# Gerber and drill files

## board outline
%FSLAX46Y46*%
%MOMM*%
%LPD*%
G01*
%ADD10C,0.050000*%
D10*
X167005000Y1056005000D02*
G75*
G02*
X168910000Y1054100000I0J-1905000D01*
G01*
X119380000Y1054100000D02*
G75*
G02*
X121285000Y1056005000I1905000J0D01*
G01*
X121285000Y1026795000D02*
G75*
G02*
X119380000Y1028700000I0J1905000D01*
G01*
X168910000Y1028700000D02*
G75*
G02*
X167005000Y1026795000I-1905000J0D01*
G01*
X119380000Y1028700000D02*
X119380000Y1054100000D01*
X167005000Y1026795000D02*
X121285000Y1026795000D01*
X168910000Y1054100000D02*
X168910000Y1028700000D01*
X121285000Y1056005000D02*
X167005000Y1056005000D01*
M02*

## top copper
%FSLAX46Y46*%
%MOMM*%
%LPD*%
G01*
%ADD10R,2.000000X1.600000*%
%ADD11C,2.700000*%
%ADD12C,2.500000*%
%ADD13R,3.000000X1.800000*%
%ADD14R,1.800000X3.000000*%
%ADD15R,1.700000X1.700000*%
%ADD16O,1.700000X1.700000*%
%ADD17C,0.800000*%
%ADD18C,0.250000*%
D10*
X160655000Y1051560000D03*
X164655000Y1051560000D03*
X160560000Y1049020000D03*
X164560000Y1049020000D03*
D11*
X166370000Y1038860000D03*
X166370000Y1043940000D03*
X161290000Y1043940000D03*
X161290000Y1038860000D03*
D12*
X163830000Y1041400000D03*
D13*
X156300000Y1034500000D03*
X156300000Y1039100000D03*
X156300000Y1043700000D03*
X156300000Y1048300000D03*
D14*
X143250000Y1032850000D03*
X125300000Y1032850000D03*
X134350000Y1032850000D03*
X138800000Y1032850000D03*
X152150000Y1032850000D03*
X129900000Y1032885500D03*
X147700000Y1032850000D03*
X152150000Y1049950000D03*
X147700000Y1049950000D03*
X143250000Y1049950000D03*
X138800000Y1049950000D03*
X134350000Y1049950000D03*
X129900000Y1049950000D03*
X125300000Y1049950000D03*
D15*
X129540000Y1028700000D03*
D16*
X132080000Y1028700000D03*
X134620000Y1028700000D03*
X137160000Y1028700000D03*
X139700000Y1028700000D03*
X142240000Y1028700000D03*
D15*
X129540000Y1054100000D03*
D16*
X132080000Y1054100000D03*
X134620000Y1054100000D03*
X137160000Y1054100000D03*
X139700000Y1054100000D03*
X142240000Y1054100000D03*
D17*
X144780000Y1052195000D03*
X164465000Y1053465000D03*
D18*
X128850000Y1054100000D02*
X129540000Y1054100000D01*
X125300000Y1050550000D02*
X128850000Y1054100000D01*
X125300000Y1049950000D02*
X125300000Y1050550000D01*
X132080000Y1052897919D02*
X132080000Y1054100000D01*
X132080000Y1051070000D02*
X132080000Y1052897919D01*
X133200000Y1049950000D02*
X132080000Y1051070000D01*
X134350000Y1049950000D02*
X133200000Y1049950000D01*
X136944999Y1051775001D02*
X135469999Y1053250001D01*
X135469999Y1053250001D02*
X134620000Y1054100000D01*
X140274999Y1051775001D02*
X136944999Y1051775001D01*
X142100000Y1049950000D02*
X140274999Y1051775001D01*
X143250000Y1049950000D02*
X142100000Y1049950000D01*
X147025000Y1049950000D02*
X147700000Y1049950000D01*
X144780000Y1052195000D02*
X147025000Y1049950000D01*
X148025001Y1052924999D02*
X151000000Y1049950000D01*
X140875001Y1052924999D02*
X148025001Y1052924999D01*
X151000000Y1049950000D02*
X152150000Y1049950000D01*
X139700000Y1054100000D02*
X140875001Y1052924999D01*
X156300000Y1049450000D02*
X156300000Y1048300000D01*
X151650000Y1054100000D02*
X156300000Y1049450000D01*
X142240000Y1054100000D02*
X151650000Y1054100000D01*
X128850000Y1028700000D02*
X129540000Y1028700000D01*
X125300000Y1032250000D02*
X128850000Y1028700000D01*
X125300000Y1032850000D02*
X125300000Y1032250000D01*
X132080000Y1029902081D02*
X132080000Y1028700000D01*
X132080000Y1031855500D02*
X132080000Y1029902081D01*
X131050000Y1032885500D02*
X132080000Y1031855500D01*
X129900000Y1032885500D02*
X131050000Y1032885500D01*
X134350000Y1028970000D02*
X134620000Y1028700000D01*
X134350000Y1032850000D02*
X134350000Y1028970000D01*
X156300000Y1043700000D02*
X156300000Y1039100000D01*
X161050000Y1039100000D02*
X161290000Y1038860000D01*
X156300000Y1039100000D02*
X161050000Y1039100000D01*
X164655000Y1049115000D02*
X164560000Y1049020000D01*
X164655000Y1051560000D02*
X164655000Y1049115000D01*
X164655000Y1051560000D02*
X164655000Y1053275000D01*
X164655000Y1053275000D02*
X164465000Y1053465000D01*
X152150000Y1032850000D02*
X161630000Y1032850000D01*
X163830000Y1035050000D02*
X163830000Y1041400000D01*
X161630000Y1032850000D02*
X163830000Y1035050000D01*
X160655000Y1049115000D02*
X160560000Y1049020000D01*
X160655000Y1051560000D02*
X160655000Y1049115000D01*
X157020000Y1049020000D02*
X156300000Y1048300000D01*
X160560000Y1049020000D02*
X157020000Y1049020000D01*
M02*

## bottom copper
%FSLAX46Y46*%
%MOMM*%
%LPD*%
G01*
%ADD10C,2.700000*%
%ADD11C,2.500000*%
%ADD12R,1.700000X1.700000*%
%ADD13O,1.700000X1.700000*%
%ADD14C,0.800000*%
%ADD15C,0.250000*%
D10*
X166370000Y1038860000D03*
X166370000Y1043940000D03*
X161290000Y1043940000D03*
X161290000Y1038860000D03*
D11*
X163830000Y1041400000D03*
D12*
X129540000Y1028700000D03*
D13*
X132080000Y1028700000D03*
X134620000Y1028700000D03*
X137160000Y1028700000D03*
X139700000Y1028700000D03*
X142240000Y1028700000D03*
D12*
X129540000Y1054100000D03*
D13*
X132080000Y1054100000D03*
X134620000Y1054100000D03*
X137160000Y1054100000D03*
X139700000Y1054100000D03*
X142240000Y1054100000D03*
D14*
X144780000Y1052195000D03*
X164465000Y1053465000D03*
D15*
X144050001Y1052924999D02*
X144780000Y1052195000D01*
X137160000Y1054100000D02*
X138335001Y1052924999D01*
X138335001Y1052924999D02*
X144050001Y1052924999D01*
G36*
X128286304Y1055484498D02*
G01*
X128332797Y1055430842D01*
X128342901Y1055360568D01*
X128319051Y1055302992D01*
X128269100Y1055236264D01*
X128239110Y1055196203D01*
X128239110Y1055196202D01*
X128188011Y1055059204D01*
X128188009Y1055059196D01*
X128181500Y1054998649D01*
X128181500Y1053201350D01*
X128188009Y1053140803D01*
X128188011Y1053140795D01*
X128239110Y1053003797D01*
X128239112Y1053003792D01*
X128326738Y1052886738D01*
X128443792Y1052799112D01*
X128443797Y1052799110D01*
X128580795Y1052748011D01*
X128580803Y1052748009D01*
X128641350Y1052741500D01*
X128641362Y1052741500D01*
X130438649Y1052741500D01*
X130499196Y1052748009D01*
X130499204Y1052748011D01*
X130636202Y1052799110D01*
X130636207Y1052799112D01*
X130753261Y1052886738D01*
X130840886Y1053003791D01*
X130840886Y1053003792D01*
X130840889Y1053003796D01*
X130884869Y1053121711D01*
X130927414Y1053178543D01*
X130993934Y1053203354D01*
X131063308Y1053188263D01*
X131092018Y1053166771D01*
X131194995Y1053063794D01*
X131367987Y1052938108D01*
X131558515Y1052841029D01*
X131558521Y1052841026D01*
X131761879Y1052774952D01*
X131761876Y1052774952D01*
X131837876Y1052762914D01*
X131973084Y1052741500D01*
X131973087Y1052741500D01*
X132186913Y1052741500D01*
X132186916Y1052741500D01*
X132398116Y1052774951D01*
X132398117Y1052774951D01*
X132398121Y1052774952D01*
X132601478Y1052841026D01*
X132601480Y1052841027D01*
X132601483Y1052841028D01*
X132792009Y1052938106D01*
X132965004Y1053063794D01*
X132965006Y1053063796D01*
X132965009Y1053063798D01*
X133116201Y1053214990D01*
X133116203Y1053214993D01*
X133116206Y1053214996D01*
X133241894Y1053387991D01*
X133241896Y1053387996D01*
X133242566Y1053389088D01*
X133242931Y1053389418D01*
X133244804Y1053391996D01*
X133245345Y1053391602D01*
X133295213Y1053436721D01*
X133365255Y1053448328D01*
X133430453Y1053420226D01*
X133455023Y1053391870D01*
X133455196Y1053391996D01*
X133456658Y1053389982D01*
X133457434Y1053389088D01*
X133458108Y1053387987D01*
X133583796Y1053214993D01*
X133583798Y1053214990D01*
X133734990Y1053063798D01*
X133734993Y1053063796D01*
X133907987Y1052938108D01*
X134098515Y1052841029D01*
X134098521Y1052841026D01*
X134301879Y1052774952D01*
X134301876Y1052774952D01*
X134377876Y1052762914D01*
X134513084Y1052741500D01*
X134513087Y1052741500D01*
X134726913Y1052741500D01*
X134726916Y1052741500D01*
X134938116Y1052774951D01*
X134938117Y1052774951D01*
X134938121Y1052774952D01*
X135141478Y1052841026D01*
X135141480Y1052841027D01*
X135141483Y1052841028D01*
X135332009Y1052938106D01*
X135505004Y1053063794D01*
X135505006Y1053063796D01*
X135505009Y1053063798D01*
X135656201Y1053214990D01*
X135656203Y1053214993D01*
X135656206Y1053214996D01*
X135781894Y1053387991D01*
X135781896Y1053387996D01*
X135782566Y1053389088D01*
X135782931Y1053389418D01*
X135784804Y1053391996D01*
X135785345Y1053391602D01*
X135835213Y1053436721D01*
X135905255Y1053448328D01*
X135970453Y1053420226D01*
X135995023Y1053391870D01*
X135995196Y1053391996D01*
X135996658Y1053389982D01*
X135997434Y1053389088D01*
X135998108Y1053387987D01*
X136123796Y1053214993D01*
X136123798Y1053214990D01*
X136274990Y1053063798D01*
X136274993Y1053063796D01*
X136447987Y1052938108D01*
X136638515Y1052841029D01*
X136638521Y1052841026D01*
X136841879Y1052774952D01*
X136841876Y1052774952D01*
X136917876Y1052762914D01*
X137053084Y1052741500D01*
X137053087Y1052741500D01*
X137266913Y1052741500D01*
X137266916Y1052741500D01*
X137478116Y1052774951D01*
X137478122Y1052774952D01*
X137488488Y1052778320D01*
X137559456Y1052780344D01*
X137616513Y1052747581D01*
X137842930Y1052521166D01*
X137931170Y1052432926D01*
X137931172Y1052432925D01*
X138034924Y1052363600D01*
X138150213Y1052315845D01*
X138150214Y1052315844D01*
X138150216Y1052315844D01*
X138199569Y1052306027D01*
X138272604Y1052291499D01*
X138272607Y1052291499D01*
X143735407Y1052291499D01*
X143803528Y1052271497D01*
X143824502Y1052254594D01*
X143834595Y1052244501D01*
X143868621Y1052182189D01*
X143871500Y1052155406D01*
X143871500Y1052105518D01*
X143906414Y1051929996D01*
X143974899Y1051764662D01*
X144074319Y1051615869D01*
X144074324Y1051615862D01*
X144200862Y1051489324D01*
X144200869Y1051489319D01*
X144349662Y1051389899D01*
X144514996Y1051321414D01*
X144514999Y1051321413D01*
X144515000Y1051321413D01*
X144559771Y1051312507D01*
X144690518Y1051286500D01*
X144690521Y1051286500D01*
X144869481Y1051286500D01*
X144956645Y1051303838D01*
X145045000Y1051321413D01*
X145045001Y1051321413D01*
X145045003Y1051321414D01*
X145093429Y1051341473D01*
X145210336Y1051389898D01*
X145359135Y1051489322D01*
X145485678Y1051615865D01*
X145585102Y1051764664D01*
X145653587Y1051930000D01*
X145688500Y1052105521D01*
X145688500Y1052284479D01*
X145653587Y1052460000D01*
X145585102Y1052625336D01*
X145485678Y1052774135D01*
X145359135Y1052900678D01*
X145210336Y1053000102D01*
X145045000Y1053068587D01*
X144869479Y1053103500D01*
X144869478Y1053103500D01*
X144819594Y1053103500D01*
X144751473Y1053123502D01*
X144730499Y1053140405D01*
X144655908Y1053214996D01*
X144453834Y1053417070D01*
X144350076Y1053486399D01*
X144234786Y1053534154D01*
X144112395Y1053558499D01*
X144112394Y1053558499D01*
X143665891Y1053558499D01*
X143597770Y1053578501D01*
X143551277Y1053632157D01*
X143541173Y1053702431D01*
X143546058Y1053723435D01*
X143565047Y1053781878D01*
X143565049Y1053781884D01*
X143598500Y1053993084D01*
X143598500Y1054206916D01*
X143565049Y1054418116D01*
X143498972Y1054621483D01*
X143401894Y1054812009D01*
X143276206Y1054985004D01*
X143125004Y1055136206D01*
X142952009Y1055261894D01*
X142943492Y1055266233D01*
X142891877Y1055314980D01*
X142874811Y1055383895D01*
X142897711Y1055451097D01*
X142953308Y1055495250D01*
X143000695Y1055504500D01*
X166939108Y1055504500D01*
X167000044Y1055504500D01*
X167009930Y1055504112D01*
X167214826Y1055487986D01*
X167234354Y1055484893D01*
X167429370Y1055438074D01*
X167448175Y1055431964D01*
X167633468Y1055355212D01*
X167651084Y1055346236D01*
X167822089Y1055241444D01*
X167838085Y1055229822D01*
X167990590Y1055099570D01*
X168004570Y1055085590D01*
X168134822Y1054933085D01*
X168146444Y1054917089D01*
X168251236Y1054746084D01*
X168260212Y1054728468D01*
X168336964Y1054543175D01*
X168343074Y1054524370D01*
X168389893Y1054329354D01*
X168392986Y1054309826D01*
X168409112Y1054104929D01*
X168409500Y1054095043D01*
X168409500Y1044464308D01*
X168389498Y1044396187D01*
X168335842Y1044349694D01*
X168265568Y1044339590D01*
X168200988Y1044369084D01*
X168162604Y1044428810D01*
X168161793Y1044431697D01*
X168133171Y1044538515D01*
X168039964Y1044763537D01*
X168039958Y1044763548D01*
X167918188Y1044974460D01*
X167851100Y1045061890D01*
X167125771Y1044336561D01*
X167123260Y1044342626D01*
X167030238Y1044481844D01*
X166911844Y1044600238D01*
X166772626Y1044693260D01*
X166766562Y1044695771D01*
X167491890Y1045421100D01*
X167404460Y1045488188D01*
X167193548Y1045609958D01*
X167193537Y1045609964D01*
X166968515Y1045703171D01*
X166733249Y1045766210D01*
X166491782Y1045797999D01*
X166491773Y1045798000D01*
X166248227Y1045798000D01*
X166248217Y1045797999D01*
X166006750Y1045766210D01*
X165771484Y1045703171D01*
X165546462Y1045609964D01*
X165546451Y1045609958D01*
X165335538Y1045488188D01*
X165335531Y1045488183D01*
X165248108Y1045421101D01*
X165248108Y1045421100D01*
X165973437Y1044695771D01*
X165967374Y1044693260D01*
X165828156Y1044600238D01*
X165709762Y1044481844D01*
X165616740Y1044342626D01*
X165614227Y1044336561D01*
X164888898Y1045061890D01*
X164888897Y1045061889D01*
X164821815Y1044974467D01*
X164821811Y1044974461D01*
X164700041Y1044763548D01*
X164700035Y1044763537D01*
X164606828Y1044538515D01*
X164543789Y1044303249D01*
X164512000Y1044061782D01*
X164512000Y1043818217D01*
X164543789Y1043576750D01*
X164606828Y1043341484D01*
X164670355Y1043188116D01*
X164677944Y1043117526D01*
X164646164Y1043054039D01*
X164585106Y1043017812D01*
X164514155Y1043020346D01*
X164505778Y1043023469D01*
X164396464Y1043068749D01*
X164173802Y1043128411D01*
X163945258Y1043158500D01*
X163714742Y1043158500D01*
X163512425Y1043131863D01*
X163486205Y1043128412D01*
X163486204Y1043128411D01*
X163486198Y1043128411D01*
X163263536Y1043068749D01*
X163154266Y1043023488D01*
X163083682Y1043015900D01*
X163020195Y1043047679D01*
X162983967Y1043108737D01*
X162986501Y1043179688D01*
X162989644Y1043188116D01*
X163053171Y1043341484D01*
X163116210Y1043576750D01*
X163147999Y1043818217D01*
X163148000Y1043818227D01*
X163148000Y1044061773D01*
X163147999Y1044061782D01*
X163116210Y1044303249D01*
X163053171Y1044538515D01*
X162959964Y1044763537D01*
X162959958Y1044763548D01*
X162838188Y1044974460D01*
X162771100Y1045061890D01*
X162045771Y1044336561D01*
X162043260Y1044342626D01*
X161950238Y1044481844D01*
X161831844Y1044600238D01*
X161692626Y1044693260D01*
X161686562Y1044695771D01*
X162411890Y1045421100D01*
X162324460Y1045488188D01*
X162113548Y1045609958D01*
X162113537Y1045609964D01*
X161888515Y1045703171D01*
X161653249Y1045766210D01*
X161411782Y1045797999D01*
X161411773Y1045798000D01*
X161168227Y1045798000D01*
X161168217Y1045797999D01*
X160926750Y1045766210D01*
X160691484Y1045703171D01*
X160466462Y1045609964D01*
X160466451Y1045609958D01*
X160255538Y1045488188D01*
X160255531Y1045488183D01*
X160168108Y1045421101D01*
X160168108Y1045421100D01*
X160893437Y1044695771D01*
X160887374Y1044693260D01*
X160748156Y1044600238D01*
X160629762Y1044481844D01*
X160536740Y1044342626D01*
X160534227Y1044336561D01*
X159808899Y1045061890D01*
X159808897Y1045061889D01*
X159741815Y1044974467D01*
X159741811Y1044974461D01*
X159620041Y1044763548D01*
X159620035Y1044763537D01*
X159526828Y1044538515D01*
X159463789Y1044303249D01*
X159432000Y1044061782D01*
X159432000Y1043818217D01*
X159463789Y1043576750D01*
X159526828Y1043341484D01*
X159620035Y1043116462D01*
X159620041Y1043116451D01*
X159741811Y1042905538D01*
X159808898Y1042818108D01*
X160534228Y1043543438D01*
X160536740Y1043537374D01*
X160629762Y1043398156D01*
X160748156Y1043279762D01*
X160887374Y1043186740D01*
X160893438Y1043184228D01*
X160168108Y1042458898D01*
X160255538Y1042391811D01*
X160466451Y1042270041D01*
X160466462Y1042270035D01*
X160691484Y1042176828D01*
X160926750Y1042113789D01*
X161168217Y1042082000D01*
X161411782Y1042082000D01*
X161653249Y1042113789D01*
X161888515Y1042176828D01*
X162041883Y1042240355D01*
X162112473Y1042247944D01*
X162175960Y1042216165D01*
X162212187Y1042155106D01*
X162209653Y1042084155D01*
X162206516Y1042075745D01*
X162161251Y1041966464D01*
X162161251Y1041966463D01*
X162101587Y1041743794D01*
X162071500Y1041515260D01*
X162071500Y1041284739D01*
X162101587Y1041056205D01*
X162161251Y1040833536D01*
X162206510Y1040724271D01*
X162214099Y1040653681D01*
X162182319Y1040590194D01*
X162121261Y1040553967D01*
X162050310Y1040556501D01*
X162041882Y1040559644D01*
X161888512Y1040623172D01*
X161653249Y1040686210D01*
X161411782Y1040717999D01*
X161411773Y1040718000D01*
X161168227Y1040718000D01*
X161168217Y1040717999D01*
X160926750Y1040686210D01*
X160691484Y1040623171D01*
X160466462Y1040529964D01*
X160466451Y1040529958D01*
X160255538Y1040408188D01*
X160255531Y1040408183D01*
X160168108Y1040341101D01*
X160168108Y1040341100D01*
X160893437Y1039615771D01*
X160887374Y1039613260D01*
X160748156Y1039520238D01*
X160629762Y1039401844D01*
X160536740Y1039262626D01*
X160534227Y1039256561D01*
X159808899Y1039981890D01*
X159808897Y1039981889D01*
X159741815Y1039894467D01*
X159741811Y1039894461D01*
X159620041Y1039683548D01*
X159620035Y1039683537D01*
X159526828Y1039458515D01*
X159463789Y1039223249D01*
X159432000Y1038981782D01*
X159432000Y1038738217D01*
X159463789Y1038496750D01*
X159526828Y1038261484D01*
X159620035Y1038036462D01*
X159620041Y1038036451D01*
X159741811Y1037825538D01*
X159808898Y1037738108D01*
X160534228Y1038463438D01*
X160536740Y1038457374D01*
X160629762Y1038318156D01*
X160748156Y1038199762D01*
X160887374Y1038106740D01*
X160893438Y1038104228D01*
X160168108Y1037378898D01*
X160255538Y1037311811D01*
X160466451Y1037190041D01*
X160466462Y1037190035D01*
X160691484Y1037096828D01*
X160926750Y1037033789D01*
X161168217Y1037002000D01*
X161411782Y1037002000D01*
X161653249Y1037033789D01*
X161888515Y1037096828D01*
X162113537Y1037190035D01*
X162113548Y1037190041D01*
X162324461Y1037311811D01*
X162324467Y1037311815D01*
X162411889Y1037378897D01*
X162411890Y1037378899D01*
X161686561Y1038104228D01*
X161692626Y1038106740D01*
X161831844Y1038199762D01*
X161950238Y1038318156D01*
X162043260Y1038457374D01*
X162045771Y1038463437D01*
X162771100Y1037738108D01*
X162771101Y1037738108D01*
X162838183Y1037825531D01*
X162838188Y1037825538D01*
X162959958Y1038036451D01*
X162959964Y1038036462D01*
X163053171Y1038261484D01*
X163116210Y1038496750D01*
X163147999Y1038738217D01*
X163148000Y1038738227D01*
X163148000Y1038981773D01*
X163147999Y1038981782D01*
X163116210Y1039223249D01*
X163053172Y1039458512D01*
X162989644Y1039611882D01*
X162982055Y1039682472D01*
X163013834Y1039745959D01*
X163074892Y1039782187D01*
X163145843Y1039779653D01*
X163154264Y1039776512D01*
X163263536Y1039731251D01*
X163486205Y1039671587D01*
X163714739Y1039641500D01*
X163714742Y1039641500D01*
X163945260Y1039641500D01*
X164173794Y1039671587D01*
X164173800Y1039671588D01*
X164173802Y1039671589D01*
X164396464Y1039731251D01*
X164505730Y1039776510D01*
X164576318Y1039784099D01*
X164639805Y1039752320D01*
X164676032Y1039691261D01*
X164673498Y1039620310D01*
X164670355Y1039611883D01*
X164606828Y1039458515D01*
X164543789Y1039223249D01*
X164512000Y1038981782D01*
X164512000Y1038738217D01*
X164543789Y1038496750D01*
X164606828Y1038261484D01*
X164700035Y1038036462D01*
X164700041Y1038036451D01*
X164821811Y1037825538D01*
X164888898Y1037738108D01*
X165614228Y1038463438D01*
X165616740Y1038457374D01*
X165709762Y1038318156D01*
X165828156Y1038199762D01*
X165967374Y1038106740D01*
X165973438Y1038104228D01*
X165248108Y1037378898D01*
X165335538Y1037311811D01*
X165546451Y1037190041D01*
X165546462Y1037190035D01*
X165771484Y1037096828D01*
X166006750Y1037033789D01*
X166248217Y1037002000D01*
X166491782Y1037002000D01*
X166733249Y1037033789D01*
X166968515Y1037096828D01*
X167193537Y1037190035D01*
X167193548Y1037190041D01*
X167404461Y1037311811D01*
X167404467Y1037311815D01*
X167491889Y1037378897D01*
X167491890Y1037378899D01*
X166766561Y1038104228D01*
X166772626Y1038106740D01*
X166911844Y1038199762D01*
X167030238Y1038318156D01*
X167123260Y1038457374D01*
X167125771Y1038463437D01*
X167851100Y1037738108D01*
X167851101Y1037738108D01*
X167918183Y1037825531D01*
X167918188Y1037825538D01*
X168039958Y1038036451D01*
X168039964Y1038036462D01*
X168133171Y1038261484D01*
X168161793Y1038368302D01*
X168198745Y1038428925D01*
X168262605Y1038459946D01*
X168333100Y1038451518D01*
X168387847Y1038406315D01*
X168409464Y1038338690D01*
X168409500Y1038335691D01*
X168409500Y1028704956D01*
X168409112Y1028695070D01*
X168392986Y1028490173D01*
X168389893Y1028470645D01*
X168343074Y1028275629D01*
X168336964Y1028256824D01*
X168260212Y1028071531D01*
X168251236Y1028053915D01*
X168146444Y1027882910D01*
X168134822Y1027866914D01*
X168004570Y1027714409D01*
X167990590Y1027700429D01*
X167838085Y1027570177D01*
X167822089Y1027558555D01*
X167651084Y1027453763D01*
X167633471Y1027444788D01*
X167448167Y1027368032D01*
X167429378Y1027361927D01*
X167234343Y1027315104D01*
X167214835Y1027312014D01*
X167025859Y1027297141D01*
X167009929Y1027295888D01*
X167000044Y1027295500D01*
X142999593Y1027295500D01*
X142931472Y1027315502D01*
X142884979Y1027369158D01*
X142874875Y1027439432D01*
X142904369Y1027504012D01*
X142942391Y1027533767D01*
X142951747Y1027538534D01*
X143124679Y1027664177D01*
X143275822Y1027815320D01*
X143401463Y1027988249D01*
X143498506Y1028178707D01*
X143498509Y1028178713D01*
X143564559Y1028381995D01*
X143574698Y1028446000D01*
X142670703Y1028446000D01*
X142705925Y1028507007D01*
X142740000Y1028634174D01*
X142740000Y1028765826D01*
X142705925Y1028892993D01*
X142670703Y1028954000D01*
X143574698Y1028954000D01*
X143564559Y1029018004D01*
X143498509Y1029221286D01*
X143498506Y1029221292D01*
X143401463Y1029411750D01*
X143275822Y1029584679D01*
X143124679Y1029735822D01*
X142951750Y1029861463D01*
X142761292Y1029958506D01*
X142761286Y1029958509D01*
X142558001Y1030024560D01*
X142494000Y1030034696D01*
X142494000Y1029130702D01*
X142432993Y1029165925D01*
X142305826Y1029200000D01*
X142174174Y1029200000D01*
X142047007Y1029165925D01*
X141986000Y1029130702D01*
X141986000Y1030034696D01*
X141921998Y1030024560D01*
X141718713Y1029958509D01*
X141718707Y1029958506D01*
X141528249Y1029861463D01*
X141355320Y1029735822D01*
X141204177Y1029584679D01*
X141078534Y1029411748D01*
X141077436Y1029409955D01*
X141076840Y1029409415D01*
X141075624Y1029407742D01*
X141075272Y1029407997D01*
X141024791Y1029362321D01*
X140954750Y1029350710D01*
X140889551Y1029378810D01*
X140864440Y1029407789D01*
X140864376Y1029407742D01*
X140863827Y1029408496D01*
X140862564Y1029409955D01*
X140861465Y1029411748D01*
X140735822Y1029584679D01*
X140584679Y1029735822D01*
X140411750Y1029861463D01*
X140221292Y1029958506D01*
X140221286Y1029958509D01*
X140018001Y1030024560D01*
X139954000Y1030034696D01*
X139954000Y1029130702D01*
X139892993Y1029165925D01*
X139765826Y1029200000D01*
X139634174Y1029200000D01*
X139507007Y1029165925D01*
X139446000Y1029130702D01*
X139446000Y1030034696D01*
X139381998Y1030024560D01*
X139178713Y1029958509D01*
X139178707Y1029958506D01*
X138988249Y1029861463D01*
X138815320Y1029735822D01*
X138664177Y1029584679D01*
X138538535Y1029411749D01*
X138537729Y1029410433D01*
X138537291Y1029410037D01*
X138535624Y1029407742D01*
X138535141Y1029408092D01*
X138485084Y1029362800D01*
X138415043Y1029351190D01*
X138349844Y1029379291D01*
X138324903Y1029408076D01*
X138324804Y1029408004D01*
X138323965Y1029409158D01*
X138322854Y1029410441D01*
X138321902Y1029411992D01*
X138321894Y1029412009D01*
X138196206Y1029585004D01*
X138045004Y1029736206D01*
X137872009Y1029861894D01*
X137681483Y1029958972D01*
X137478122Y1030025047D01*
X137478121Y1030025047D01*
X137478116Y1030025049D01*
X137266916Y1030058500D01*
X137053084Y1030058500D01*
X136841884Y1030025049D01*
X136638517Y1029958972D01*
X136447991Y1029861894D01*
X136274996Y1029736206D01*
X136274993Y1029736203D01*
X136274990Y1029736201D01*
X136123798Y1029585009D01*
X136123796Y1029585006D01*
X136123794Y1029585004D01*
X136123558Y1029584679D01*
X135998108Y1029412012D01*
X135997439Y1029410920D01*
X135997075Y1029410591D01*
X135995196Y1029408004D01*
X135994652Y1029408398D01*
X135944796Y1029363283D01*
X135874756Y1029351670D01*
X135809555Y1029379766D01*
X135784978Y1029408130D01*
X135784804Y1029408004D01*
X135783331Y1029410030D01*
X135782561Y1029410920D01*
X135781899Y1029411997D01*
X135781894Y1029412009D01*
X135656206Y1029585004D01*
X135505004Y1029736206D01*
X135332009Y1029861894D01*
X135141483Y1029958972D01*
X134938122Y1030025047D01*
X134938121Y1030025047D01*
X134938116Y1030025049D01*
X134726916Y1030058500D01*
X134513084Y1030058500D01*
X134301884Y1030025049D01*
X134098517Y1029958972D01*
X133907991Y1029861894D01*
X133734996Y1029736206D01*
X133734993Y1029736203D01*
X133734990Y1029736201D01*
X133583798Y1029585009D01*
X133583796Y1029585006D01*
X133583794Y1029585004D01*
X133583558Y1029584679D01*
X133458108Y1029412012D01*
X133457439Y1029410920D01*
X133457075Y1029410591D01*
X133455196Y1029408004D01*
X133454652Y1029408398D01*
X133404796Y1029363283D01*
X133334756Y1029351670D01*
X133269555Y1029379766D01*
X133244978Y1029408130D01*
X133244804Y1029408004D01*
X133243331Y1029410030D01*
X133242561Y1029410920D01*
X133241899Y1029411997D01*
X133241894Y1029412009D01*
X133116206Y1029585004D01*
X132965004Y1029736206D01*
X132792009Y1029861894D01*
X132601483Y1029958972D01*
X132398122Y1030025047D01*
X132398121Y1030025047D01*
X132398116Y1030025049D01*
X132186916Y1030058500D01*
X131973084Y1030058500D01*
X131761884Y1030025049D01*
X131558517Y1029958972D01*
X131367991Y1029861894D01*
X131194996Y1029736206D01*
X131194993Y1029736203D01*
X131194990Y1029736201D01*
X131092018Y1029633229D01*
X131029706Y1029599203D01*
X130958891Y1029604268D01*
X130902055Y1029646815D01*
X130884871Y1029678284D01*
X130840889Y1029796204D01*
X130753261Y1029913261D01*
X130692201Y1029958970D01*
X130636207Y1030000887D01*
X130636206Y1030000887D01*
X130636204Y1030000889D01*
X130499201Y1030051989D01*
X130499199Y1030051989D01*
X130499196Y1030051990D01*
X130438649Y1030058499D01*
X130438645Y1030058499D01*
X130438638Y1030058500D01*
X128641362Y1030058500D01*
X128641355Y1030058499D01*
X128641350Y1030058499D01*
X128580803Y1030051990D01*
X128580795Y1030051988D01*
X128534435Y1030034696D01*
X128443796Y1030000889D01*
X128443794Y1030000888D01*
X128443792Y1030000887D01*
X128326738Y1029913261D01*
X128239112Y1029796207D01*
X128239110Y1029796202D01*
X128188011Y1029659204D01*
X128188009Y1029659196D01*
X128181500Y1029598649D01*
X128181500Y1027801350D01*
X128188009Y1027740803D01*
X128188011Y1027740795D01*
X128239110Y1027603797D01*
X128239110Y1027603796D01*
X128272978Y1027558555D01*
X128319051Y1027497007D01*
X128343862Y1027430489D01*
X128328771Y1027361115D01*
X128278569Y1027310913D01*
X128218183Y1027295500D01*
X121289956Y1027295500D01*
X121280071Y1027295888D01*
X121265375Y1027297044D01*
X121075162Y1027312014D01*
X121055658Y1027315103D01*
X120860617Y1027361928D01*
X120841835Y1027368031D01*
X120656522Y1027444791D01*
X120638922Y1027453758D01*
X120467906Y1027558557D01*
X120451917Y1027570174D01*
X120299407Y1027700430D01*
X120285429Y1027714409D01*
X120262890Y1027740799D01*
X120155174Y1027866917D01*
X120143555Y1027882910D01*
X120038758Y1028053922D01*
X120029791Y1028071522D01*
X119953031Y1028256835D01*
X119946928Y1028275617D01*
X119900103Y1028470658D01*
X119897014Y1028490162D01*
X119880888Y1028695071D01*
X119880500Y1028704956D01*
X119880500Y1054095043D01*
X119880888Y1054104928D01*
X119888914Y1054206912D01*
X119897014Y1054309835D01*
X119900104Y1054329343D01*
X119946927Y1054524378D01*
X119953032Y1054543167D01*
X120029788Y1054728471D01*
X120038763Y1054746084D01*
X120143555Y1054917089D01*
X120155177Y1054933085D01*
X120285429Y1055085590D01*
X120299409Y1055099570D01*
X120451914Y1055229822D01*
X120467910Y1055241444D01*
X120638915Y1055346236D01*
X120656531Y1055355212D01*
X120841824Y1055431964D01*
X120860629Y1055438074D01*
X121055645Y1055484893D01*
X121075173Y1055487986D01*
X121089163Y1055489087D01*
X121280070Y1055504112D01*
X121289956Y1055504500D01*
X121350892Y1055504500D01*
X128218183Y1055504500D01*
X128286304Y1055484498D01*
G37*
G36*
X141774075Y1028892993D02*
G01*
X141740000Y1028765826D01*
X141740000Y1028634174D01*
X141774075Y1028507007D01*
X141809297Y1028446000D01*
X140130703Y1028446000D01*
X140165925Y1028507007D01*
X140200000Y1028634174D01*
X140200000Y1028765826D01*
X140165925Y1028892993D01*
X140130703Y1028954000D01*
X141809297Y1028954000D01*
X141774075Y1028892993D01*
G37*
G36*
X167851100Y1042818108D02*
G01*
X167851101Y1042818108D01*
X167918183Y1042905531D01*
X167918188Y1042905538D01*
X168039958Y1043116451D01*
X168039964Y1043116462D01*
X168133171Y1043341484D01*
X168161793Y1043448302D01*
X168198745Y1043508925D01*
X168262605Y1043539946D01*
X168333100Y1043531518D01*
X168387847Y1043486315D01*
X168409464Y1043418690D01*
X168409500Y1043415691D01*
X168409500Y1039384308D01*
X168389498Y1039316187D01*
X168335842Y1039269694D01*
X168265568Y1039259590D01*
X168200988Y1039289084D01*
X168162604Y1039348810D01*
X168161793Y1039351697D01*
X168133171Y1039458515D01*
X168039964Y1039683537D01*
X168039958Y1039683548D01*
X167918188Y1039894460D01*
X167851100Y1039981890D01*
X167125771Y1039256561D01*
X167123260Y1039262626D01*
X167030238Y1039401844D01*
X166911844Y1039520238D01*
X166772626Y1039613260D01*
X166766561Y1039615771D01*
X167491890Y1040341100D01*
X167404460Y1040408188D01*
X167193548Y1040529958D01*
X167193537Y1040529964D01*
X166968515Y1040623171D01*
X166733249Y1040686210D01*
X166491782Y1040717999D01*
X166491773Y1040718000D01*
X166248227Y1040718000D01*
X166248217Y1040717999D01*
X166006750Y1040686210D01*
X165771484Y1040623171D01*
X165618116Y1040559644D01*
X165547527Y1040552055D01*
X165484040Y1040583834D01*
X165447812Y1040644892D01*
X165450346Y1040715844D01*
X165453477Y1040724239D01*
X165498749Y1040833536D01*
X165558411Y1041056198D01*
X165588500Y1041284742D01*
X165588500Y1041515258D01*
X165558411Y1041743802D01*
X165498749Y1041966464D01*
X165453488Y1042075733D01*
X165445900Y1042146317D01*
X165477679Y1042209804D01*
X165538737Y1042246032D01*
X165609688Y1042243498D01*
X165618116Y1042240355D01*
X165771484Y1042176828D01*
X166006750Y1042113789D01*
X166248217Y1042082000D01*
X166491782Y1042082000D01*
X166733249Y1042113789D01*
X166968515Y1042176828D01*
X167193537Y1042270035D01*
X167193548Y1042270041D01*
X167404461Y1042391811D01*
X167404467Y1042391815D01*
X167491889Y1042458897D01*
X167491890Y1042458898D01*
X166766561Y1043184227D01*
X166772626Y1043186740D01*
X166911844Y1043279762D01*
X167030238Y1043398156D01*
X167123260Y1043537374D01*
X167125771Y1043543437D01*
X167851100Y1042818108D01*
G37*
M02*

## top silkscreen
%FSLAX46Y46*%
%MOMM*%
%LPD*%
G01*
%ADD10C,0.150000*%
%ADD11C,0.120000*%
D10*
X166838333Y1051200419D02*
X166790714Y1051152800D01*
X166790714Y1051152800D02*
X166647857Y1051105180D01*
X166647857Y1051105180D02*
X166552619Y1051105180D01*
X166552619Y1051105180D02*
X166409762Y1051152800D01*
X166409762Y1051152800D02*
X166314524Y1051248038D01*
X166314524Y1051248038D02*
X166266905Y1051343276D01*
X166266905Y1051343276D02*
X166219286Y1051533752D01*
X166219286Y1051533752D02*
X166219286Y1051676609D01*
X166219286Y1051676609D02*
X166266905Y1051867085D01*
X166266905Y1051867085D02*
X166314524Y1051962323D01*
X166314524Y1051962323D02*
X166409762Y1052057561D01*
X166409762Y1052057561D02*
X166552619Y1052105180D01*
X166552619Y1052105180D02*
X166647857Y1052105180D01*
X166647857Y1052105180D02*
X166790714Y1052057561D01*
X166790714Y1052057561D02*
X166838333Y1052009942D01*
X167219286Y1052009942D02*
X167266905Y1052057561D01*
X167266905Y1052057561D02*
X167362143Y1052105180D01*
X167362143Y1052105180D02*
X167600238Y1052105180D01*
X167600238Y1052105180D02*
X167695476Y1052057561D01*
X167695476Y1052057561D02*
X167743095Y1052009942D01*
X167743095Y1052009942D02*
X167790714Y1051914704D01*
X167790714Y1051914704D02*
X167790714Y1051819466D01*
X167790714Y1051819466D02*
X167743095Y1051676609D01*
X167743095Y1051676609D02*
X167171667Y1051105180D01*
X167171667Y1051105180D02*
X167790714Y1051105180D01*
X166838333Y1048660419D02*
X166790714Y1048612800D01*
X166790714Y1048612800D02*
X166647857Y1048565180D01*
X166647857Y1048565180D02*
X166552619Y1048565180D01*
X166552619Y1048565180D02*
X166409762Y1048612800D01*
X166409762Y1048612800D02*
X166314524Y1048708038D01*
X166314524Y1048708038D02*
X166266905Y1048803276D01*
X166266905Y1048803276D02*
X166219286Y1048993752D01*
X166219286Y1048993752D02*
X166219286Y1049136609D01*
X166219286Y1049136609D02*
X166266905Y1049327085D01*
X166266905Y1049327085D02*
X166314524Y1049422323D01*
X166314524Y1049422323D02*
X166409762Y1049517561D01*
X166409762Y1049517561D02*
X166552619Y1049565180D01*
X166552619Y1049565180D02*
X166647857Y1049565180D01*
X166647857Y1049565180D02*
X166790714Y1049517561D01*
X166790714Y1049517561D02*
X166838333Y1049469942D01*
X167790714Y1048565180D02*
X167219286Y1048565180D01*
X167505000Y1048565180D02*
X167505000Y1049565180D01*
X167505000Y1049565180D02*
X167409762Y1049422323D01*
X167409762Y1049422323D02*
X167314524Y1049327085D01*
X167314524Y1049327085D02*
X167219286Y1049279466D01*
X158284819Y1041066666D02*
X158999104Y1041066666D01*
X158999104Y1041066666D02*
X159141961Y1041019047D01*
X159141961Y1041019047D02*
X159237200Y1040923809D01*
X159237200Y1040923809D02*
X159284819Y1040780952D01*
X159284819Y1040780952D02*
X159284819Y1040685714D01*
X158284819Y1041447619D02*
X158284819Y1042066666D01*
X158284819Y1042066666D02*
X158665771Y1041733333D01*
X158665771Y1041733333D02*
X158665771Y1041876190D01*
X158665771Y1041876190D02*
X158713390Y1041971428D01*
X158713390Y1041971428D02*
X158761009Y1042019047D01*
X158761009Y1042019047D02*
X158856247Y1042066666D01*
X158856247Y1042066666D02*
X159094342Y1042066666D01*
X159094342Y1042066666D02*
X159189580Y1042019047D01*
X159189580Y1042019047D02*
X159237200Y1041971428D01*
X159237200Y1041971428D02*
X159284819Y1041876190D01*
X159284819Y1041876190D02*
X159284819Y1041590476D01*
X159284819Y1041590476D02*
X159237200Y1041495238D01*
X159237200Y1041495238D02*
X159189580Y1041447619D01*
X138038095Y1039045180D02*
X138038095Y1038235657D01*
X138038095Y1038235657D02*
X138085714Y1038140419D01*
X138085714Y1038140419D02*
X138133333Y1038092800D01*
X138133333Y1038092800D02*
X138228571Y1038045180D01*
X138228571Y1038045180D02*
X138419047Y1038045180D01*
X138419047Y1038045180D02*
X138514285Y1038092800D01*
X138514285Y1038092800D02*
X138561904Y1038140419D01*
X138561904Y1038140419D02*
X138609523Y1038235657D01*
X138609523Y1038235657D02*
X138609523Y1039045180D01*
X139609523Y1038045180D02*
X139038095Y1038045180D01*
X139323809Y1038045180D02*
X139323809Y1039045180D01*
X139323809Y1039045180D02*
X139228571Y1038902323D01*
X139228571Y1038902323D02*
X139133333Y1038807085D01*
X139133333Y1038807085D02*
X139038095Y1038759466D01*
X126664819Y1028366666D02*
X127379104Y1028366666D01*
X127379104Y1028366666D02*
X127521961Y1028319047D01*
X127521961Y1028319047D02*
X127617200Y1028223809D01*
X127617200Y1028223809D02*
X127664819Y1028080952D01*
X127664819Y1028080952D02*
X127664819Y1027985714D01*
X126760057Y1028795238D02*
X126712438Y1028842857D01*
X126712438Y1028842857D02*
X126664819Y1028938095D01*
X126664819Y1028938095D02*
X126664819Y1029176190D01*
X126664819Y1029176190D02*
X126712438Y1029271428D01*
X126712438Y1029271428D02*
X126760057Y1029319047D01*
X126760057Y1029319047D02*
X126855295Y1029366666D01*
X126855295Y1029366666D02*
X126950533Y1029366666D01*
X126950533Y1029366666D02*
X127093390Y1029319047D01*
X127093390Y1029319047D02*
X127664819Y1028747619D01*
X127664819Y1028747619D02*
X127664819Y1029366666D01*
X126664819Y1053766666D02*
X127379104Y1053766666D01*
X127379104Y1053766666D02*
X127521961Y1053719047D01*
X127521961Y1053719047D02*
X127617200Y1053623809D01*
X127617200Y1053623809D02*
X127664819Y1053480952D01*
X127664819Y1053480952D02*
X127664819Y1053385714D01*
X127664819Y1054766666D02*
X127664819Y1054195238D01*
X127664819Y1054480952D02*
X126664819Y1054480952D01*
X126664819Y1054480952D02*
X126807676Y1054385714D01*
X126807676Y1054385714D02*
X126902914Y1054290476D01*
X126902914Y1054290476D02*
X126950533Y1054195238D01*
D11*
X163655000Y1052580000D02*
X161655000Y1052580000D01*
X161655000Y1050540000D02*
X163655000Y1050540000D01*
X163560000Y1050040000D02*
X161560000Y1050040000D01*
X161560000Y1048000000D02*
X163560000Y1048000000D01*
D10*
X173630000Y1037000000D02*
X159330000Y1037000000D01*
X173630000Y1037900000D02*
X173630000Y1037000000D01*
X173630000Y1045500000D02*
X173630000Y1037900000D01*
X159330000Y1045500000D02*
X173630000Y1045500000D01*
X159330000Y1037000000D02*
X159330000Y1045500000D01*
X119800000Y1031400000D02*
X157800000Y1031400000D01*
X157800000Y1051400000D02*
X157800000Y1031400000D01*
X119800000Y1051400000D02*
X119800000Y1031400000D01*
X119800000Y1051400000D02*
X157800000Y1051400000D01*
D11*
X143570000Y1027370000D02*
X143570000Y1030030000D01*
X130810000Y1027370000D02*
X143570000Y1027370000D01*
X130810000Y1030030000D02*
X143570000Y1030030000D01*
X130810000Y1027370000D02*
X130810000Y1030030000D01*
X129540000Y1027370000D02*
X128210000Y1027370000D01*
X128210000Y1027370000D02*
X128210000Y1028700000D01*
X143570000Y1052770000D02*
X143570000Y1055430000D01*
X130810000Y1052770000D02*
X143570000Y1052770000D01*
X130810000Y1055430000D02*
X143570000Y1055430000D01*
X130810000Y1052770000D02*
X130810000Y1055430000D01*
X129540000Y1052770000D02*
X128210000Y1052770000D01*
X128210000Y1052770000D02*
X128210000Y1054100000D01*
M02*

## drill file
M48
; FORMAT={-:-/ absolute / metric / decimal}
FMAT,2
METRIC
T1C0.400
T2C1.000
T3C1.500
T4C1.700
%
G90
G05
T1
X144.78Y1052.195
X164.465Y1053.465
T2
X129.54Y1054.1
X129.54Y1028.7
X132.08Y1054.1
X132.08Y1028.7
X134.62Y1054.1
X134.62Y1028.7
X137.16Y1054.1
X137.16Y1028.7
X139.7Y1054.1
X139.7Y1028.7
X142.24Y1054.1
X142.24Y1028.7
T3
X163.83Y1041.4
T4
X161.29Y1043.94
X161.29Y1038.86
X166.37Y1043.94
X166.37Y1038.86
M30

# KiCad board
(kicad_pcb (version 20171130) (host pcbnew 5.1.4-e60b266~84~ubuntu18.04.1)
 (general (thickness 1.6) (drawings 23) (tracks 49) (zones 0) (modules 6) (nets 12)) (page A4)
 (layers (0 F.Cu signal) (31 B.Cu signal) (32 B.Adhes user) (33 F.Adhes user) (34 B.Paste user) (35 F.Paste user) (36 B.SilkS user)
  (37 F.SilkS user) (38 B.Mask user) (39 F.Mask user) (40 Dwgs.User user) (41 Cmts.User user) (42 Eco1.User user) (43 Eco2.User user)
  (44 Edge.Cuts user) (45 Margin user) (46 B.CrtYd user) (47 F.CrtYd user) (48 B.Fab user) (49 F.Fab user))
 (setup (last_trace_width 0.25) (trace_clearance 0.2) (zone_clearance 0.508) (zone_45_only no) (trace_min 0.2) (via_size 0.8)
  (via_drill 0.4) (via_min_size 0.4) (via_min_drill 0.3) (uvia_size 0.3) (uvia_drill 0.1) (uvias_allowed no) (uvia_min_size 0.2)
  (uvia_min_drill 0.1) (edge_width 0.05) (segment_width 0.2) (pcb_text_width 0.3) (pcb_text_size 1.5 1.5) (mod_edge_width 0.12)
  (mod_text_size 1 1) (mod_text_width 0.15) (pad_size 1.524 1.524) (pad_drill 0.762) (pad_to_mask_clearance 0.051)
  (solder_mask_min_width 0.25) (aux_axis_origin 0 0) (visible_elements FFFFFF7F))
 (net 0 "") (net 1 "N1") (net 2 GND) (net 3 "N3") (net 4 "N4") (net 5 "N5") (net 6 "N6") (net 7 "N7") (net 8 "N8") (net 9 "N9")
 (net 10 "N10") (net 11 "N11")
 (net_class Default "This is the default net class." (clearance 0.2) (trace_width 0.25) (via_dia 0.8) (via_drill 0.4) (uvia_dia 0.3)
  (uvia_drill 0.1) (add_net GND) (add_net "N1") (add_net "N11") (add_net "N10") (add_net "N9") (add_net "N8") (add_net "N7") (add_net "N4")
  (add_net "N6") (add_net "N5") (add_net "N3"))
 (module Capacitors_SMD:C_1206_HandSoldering (layer F.Cu) (at 162.655 -1051.56)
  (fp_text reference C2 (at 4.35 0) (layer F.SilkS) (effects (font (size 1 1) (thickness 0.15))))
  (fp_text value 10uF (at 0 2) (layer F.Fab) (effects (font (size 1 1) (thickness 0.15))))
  (fp_line (start 1 -1.02) (end -1 -1.02) (layer F.SilkS) (width 0.12))
  (fp_line (start -1 1.02) (end 1 1.02) (layer F.SilkS) (width 0.12))
  (pad 1 smd rect (at -2 0) (size 2 1.6) (layers F.Cu F.Paste F.Mask) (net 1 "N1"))
  (pad 2 smd rect (at 2 0) (size 2 1.6) (layers F.Cu F.Paste F.Mask) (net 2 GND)))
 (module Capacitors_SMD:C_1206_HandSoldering (layer F.Cu) (at 162.56 -1049.02)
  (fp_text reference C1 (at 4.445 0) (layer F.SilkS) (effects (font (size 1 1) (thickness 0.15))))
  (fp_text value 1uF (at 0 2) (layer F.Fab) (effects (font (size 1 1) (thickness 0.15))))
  (fp_line (start 1 -1.02) (end -1 -1.02) (layer F.SilkS) (width 0.12))
  (fp_line (start -1 1.02) (end 1 1.02) (layer F.SilkS) (width 0.12))
  (pad 1 smd rect (at -2 0) (size 2 1.6) (layers F.Cu F.Paste F.Mask) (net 1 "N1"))
  (pad 2 smd rect (at 2 0) (size 2 1.6) (layers F.Cu F.Paste F.Mask) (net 2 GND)))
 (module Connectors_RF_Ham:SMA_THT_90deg (layer F.Cu) (at 163.83 -1041.4 90)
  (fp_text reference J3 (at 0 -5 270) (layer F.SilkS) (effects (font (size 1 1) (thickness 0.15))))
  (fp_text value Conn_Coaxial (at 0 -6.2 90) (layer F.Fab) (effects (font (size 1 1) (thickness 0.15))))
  (fp_line (start -4.4 9.8) (end -4.4 -4.5) (layer F.SilkS) (width 0.15))
  (fp_line (start -3.5 9.8) (end -4.4 9.8) (layer F.SilkS) (width 0.15))
  (fp_line (start 4.1 9.8) (end -3.5 9.8) (layer F.SilkS) (width 0.15))
  (fp_line (start 4.1 -4.5) (end 4.1 9.8) (layer F.SilkS) (width 0.15))
  (fp_line (start -4.4 -4.5) (end 4.1 -4.5) (layer F.SilkS) (width 0.15))
  (pad 2 thru_hole circle (at -2.54 2.54 90) (size 2.7 2.7) (drill 1.7) (layers *.Cu *.Mask) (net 2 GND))
  (pad 2 thru_hole circle (at 2.54 2.54 90) (size 2.7 2.7) (drill 1.7) (layers *.Cu *.Mask) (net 2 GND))
  (pad 2 thru_hole circle (at 2.54 -2.54 90) (size 2.7 2.7) (drill 1.7) (layers *.Cu *.Mask) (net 2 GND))
  (pad 2 thru_hole circle (at -2.54 -2.54 90) (size 2.7 2.7) (drill 1.7) (layers *.Cu *.Mask) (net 2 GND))
  (pad 1 thru_hole circle (at 0 0 90) (size 2.5 2.5) (drill 1.5) (layers *.Cu *.Mask) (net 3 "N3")))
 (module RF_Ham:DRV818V (layer F.Cu) (at 138.8 -1041.4)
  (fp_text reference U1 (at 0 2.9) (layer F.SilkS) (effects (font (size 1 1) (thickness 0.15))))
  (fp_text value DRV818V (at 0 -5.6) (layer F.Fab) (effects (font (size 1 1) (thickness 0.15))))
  (fp_line (start -19 10) (end 19 10) (layer F.SilkS) (width 0.15))
  (fp_line (start 19 -10) (end 19 10) (layer F.SilkS) (width 0.15))
  (fp_line (start -19 -10) (end -19 10) (layer F.SilkS) (width 0.15))
  (fp_line (start -19 -10) (end 19 -10) (layer F.SilkS) (width 0.15))
  (pad 11 smd rect (at 17.5 6.9 90) (size 1.8 3) (layers F.Cu F.Paste F.Mask))
  (pad 10 smd rect (at 17.5 2.3 90) (size 1.8 3) (layers F.Cu F.Paste F.Mask) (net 2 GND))
  (pad 9 smd rect (at 17.5 -2.3 90) (size 1.8 3) (layers F.Cu F.Paste F.Mask) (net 2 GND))
  (pad 8 smd rect (at 17.5 -6.9 90) (size 1.8 3) (layers F.Cu F.Paste F.Mask) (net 1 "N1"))
  (pad 14 smd rect (at 4.45 8.55) (size 1.8 3) (layers F.Cu F.Paste F.Mask))
  (pad 18 smd rect (at -13.5 8.55) (size 1.8 3) (layers F.Cu F.Paste F.Mask) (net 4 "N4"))
  (pad 16 smd rect (at -4.45 8.55) (size 1.8 3) (layers F.Cu F.Paste F.Mask) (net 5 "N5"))
  (pad 15 smd rect (at 0 8.55) (size 1.8 3) (layers F.Cu F.Paste F.Mask))
  (pad 12 smd rect (at 13.35 8.55) (size 1.8 3) (layers F.Cu F.Paste F.Mask) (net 3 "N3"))
  (pad 17 smd rect (at -8.9 8.5145) (size 1.8 3) (layers F.Cu F.Paste F.Mask) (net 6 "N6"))
  (pad 13 smd rect (at 8.9 8.55) (size 1.8 3) (layers F.Cu F.Paste F.Mask))
  (pad 7 smd rect (at 13.35 -8.55) (size 1.8 3) (layers F.Cu F.Paste F.Mask) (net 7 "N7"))
  (pad 6 smd rect (at 8.9 -8.55) (size 1.8 3) (layers F.Cu F.Paste F.Mask) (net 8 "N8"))
  (pad 5 smd rect (at 4.45 -8.55) (size 1.8 3) (layers F.Cu F.Paste F.Mask) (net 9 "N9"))
  (pad 4 smd rect (at 0 -8.55) (size 1.8 3) (layers F.Cu F.Paste F.Mask))
  (pad 3 smd rect (at -4.45 -8.55) (size 1.8 3) (layers F.Cu F.Paste F.Mask) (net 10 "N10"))
  (pad 2 smd rect (at -8.9 -8.55) (size 1.8 3) (layers F.Cu F.Paste F.Mask))
  (pad 1 smd rect (at -13.5 -8.55) (size 1.8 3) (layers F.Cu F.Paste F.Mask) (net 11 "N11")))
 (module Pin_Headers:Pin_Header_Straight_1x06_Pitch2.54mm (layer F.Cu) (at 129.54 -1028.7 90)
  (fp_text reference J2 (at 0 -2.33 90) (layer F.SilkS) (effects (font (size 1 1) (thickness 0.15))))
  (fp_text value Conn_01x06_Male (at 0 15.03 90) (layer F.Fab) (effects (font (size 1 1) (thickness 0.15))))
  (fp_line (start -1.33 14.03) (end 1.33 14.03) (layer F.SilkS) (width 0.12))
  (fp_line (start -1.33 1.27) (end -1.33 14.03) (layer F.SilkS) (width 0.12))
  (fp_line (start 1.33 1.27) (end 1.33 14.03) (layer F.SilkS) (width 0.12))
  (fp_line (start -1.33 1.27) (end 1.33 1.27) (layer F.SilkS) (width 0.12))
  (fp_line (start -1.33 0) (end -1.33 -1.33) (layer F.SilkS) (width 0.12))
  (fp_line (start -1.33 -1.33) (end 0 -1.33) (layer F.SilkS) (width 0.12))
  (pad 1 thru_hole rect (at 0 0 90) (size 1.7 1.7) (drill 1) (layers *.Cu *.Mask) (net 4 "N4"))
  (pad 2 thru_hole oval (at 0 2.54 90) (size 1.7 1.7) (drill 1) (layers *.Cu *.Mask) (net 6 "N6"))
  (pad 3 thru_hole oval (at 0 5.08 90) (size 1.7 1.7) (drill 1) (layers *.Cu *.Mask) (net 5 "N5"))
  (pad 4 thru_hole oval (at 0 7.62 90) (size 1.7 1.7) (drill 1) (layers *.Cu *.Mask))
  (pad 5 thru_hole oval (at 0 10.16 90) (size 1.7 1.7) (drill 1) (layers *.Cu *.Mask) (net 2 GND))
  (pad 6 thru_hole oval (at 0 12.7 90) (size 1.7 1.7) (drill 1) (layers *.Cu *.Mask) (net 2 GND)))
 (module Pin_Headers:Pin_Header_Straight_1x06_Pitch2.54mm (layer F.Cu) (at 129.54 -1054.1 90)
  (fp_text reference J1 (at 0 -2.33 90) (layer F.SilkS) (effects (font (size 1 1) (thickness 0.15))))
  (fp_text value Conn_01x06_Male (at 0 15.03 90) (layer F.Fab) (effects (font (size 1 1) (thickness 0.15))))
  (fp_line (start -1.33 14.03) (end 1.33 14.03) (layer F.SilkS) (width 0.12))
  (fp_line (start -1.33 1.27) (end -1.33 14.03) (layer F.SilkS) (width 0.12))
  (fp_line (start 1.33 1.27) (end 1.33 14.03) (layer F.SilkS) (width 0.12))
  (fp_line (start -1.33 1.27) (end 1.33 1.27) (layer F.SilkS) (width 0.12))
  (fp_line (start -1.33 0) (end -1.33 -1.33) (layer F.SilkS) (width 0.12))
  (fp_line (start -1.33 -1.33) (end 0 -1.33) (layer F.SilkS) (width 0.12))
  (pad 1 thru_hole rect (at 0 0 90) (size 1.7 1.7) (drill 1) (layers *.Cu *.Mask) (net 11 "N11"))
  (pad 2 thru_hole oval (at 0 2.54 90) (size 1.7 1.7) (drill 1) (layers *.Cu *.Mask) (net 10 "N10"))
  (pad 3 thru_hole oval (at 0 5.08 90) (size 1.7 1.7) (drill 1) (layers *.Cu *.Mask) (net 9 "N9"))
  (pad 4 thru_hole oval (at 0 7.62 90) (size 1.7 1.7) (drill 1) (layers *.Cu *.Mask) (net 8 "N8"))
  (pad 5 thru_hole oval (at 0 10.16 90) (size 1.7 1.7) (drill 1) (layers *.Cu *.Mask) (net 7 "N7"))
  (pad 6 thru_hole oval (at 0 12.7 90) (size 1.7 1.7) (drill 1) (layers *.Cu *.Mask) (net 1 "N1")))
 (gr_arc (start 167.005 -1054.1) (end 168.91 -1054.1) (angle -90) (layer Edge.Cuts) (width 0.05))
 (gr_arc (start 121.285 -1054.1) (end 121.285 -1056.005) (angle -90) (layer Edge.Cuts) (width 0.05))
 (gr_arc (start 121.285 -1028.7) (end 119.38 -1028.7) (angle -90) (layer Edge.Cuts) (width 0.05))
 (gr_arc (start 167.005 -1028.7) (end 167.005 -1026.795) (angle -90) (layer Edge.Cuts) (width 0.05))
 (gr_line (start 119.38 -1028.7) (end 119.38 -1054.1) (layer Edge.Cuts) (width 0.05))
 (gr_line (start 167.005 -1026.795) (end 121.285 -1026.795) (layer Edge.Cuts) (width 0.05))
 (gr_line (start 168.91 -1054.1) (end 168.91 -1028.7) (layer Edge.Cuts) (width 0.05))
 (gr_line (start 121.285 -1056.005) (end 167.005 -1056.005) (layer Edge.Cuts) (width 0.05))
 (segment (start 128.85 -1054.1) (end 129.54 -1054.1) (width 0.25) (layer F.Cu) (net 11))
 (segment (start 125.3 -1050.55) (end 128.85 -1054.1) (width 0.25) (layer F.Cu) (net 11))
 (segment (start 125.3 -1049.95) (end 125.3 -1050.55) (width 0.25) (layer F.Cu) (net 11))
 (segment (start 132.08 -1052.897919) (end 132.08 -1054.1) (width 0.25) (layer F.Cu) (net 10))
 (segment (start 132.08 -1051.07) (end 132.08 -1052.897919) (width 0.25) (layer F.Cu) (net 10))
 (segment (start 133.2 -1049.95) (end 132.08 -1051.07) (width 0.25) (layer F.Cu) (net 10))
 (segment (start 134.35 -1049.95) (end 133.2 -1049.95) (width 0.25) (layer F.Cu) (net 10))
 (segment (start 136.944999 -1051.775001) (end 135.469999 -1053.250001) (width 0.25) (layer F.Cu) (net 9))
 (segment (start 135.469999 -1053.250001) (end 134.62 -1054.1) (width 0.25) (layer F.Cu) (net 9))
 (segment (start 140.274999 -1051.775001) (end 136.944999 -1051.775001) (width 0.25) (layer F.Cu) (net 9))
 (segment (start 142.1 -1049.95) (end 140.274999 -1051.775001) (width 0.25) (layer F.Cu) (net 9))
 (segment (start 143.25 -1049.95) (end 142.1 -1049.95) (width 0.25) (layer F.Cu) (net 9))
 (via (at 144.78 -1052.195) (size 0.8) (drill 0.4) (layers F.Cu B.Cu) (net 8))
 (segment (start 144.050001 -1052.924999) (end 144.78 -1052.195) (width 0.25) (layer B.Cu) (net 8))
 (segment (start 137.16 -1054.1) (end 138.335001 -1052.924999) (width 0.25) (layer B.Cu) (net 8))
 (segment (start 138.335001 -1052.924999) (end 144.050001 -1052.924999) (width 0.25) (layer B.Cu) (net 8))
 (segment (start 147.025 -1049.95) (end 147.7 -1049.95) (width 0.25) (layer F.Cu) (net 8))
 (segment (start 144.78 -1052.195) (end 147.025 -1049.95) (width 0.25) (layer F.Cu) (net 8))
 (segment (start 148.025001 -1052.924999) (end 151 -1049.95) (width 0.25) (layer F.Cu) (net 7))
 (segment (start 140.875001 -1052.924999) (end 148.025001 -1052.924999) (width 0.25) (layer F.Cu) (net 7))
 (segment (start 151 -1049.95) (end 152.15 -1049.95) (width 0.25) (layer F.Cu) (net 7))
 (segment (start 139.7 -1054.1) (end 140.875001 -1052.924999) (width 0.25) (layer F.Cu) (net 7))
 (segment (start 156.3 -1049.45) (end 156.3 -1048.3) (width 0.25) (layer F.Cu) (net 1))
 (segment (start 151.65 -1054.1) (end 156.3 -1049.45) (width 0.25) (layer F.Cu) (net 1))
 (segment (start 142.24 -1054.1) (end 151.65 -1054.1) (width 0.25) (layer F.Cu) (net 1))
 (segment (start 128.85 -1028.7) (end 129.54 -1028.7) (width 0.25) (layer F.Cu) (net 4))
 (segment (start 125.3 -1032.25) (end 128.85 -1028.7) (width 0.25) (layer F.Cu) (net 4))
 (segment (start 125.3 -1032.85) (end 125.3 -1032.25) (width 0.25) (layer F.Cu) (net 4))
 (segment (start 132.08 -1029.902081) (end 132.08 -1028.7) (width 0.25) (layer F.Cu) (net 6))
 (segment (start 132.08 -1031.8555) (end 132.08 -1029.902081) (width 0.25) (layer F.Cu) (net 6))
 (segment (start 131.05 -1032.8855) (end 132.08 -1031.8555) (width 0.25) (layer F.Cu) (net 6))
 (segment (start 129.9 -1032.8855) (end 131.05 -1032.8855) (width 0.25) (layer F.Cu) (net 6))
 (segment (start 134.35 -1028.97) (end 134.62 -1028.7) (width 0.25) (layer F.Cu) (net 5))
 (segment (start 134.35 -1032.85) (end 134.35 -1028.97) (width 0.25) (layer F.Cu) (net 5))
 (segment (start 156.3 -1043.7) (end 156.3 -1039.1) (width 0.25) (layer F.Cu) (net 2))
 (segment (start 161.05 -1039.1) (end 161.29 -1038.86) (width 0.25) (layer F.Cu) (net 2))
 (segment (start 156.3 -1039.1) (end 161.05 -1039.1) (width 0.25) (layer F.Cu) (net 2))
 (segment (start 164.655 -1049.115) (end 164.56 -1049.02) (width 0.25) (layer F.Cu) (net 2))
 (segment (start 164.655 -1051.56) (end 164.655 -1049.115) (width 0.25) (layer F.Cu) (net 2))
 (via (at 164.465 -1053.465) (size 0.8) (drill 0.4) (layers F.Cu B.Cu) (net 2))
 (segment (start 164.655 -1051.56) (end 164.655 -1053.275) (width 0.25) (layer F.Cu) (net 2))
 (segment (start 164.655 -1053.275) (end 164.465 -1053.465) (width 0.25) (layer F.Cu) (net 2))
 (segment (start 152.15 -1032.85) (end 161.63 -1032.85) (width 0.25) (layer F.Cu) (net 3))
 (segment (start 163.83 -1035.05) (end 163.83 -1041.4) (width 0.25) (layer F.Cu) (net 3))
 (segment (start 161.63 -1032.85) (end 163.83 -1035.05) (width 0.25) (layer F.Cu) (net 3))
 (segment (start 160.655 -1049.115) (end 160.56 -1049.02) (width 0.25) (layer F.Cu) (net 1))
 (segment (start 160.655 -1051.56) (end 160.655 -1049.115) (width 0.25) (layer F.Cu) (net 1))
 (segment (start 157.02 -1049.02) (end 156.3 -1048.3) (width 0.25) (layer F.Cu) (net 1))
 (segment (start 160.56 -1049.02) (end 157.02 -1049.02) (width 0.25) (layer F.Cu) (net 1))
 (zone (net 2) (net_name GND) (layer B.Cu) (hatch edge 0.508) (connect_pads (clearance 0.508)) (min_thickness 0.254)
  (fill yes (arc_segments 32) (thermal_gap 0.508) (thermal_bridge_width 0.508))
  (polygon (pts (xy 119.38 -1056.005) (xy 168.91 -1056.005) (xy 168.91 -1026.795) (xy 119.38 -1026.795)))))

